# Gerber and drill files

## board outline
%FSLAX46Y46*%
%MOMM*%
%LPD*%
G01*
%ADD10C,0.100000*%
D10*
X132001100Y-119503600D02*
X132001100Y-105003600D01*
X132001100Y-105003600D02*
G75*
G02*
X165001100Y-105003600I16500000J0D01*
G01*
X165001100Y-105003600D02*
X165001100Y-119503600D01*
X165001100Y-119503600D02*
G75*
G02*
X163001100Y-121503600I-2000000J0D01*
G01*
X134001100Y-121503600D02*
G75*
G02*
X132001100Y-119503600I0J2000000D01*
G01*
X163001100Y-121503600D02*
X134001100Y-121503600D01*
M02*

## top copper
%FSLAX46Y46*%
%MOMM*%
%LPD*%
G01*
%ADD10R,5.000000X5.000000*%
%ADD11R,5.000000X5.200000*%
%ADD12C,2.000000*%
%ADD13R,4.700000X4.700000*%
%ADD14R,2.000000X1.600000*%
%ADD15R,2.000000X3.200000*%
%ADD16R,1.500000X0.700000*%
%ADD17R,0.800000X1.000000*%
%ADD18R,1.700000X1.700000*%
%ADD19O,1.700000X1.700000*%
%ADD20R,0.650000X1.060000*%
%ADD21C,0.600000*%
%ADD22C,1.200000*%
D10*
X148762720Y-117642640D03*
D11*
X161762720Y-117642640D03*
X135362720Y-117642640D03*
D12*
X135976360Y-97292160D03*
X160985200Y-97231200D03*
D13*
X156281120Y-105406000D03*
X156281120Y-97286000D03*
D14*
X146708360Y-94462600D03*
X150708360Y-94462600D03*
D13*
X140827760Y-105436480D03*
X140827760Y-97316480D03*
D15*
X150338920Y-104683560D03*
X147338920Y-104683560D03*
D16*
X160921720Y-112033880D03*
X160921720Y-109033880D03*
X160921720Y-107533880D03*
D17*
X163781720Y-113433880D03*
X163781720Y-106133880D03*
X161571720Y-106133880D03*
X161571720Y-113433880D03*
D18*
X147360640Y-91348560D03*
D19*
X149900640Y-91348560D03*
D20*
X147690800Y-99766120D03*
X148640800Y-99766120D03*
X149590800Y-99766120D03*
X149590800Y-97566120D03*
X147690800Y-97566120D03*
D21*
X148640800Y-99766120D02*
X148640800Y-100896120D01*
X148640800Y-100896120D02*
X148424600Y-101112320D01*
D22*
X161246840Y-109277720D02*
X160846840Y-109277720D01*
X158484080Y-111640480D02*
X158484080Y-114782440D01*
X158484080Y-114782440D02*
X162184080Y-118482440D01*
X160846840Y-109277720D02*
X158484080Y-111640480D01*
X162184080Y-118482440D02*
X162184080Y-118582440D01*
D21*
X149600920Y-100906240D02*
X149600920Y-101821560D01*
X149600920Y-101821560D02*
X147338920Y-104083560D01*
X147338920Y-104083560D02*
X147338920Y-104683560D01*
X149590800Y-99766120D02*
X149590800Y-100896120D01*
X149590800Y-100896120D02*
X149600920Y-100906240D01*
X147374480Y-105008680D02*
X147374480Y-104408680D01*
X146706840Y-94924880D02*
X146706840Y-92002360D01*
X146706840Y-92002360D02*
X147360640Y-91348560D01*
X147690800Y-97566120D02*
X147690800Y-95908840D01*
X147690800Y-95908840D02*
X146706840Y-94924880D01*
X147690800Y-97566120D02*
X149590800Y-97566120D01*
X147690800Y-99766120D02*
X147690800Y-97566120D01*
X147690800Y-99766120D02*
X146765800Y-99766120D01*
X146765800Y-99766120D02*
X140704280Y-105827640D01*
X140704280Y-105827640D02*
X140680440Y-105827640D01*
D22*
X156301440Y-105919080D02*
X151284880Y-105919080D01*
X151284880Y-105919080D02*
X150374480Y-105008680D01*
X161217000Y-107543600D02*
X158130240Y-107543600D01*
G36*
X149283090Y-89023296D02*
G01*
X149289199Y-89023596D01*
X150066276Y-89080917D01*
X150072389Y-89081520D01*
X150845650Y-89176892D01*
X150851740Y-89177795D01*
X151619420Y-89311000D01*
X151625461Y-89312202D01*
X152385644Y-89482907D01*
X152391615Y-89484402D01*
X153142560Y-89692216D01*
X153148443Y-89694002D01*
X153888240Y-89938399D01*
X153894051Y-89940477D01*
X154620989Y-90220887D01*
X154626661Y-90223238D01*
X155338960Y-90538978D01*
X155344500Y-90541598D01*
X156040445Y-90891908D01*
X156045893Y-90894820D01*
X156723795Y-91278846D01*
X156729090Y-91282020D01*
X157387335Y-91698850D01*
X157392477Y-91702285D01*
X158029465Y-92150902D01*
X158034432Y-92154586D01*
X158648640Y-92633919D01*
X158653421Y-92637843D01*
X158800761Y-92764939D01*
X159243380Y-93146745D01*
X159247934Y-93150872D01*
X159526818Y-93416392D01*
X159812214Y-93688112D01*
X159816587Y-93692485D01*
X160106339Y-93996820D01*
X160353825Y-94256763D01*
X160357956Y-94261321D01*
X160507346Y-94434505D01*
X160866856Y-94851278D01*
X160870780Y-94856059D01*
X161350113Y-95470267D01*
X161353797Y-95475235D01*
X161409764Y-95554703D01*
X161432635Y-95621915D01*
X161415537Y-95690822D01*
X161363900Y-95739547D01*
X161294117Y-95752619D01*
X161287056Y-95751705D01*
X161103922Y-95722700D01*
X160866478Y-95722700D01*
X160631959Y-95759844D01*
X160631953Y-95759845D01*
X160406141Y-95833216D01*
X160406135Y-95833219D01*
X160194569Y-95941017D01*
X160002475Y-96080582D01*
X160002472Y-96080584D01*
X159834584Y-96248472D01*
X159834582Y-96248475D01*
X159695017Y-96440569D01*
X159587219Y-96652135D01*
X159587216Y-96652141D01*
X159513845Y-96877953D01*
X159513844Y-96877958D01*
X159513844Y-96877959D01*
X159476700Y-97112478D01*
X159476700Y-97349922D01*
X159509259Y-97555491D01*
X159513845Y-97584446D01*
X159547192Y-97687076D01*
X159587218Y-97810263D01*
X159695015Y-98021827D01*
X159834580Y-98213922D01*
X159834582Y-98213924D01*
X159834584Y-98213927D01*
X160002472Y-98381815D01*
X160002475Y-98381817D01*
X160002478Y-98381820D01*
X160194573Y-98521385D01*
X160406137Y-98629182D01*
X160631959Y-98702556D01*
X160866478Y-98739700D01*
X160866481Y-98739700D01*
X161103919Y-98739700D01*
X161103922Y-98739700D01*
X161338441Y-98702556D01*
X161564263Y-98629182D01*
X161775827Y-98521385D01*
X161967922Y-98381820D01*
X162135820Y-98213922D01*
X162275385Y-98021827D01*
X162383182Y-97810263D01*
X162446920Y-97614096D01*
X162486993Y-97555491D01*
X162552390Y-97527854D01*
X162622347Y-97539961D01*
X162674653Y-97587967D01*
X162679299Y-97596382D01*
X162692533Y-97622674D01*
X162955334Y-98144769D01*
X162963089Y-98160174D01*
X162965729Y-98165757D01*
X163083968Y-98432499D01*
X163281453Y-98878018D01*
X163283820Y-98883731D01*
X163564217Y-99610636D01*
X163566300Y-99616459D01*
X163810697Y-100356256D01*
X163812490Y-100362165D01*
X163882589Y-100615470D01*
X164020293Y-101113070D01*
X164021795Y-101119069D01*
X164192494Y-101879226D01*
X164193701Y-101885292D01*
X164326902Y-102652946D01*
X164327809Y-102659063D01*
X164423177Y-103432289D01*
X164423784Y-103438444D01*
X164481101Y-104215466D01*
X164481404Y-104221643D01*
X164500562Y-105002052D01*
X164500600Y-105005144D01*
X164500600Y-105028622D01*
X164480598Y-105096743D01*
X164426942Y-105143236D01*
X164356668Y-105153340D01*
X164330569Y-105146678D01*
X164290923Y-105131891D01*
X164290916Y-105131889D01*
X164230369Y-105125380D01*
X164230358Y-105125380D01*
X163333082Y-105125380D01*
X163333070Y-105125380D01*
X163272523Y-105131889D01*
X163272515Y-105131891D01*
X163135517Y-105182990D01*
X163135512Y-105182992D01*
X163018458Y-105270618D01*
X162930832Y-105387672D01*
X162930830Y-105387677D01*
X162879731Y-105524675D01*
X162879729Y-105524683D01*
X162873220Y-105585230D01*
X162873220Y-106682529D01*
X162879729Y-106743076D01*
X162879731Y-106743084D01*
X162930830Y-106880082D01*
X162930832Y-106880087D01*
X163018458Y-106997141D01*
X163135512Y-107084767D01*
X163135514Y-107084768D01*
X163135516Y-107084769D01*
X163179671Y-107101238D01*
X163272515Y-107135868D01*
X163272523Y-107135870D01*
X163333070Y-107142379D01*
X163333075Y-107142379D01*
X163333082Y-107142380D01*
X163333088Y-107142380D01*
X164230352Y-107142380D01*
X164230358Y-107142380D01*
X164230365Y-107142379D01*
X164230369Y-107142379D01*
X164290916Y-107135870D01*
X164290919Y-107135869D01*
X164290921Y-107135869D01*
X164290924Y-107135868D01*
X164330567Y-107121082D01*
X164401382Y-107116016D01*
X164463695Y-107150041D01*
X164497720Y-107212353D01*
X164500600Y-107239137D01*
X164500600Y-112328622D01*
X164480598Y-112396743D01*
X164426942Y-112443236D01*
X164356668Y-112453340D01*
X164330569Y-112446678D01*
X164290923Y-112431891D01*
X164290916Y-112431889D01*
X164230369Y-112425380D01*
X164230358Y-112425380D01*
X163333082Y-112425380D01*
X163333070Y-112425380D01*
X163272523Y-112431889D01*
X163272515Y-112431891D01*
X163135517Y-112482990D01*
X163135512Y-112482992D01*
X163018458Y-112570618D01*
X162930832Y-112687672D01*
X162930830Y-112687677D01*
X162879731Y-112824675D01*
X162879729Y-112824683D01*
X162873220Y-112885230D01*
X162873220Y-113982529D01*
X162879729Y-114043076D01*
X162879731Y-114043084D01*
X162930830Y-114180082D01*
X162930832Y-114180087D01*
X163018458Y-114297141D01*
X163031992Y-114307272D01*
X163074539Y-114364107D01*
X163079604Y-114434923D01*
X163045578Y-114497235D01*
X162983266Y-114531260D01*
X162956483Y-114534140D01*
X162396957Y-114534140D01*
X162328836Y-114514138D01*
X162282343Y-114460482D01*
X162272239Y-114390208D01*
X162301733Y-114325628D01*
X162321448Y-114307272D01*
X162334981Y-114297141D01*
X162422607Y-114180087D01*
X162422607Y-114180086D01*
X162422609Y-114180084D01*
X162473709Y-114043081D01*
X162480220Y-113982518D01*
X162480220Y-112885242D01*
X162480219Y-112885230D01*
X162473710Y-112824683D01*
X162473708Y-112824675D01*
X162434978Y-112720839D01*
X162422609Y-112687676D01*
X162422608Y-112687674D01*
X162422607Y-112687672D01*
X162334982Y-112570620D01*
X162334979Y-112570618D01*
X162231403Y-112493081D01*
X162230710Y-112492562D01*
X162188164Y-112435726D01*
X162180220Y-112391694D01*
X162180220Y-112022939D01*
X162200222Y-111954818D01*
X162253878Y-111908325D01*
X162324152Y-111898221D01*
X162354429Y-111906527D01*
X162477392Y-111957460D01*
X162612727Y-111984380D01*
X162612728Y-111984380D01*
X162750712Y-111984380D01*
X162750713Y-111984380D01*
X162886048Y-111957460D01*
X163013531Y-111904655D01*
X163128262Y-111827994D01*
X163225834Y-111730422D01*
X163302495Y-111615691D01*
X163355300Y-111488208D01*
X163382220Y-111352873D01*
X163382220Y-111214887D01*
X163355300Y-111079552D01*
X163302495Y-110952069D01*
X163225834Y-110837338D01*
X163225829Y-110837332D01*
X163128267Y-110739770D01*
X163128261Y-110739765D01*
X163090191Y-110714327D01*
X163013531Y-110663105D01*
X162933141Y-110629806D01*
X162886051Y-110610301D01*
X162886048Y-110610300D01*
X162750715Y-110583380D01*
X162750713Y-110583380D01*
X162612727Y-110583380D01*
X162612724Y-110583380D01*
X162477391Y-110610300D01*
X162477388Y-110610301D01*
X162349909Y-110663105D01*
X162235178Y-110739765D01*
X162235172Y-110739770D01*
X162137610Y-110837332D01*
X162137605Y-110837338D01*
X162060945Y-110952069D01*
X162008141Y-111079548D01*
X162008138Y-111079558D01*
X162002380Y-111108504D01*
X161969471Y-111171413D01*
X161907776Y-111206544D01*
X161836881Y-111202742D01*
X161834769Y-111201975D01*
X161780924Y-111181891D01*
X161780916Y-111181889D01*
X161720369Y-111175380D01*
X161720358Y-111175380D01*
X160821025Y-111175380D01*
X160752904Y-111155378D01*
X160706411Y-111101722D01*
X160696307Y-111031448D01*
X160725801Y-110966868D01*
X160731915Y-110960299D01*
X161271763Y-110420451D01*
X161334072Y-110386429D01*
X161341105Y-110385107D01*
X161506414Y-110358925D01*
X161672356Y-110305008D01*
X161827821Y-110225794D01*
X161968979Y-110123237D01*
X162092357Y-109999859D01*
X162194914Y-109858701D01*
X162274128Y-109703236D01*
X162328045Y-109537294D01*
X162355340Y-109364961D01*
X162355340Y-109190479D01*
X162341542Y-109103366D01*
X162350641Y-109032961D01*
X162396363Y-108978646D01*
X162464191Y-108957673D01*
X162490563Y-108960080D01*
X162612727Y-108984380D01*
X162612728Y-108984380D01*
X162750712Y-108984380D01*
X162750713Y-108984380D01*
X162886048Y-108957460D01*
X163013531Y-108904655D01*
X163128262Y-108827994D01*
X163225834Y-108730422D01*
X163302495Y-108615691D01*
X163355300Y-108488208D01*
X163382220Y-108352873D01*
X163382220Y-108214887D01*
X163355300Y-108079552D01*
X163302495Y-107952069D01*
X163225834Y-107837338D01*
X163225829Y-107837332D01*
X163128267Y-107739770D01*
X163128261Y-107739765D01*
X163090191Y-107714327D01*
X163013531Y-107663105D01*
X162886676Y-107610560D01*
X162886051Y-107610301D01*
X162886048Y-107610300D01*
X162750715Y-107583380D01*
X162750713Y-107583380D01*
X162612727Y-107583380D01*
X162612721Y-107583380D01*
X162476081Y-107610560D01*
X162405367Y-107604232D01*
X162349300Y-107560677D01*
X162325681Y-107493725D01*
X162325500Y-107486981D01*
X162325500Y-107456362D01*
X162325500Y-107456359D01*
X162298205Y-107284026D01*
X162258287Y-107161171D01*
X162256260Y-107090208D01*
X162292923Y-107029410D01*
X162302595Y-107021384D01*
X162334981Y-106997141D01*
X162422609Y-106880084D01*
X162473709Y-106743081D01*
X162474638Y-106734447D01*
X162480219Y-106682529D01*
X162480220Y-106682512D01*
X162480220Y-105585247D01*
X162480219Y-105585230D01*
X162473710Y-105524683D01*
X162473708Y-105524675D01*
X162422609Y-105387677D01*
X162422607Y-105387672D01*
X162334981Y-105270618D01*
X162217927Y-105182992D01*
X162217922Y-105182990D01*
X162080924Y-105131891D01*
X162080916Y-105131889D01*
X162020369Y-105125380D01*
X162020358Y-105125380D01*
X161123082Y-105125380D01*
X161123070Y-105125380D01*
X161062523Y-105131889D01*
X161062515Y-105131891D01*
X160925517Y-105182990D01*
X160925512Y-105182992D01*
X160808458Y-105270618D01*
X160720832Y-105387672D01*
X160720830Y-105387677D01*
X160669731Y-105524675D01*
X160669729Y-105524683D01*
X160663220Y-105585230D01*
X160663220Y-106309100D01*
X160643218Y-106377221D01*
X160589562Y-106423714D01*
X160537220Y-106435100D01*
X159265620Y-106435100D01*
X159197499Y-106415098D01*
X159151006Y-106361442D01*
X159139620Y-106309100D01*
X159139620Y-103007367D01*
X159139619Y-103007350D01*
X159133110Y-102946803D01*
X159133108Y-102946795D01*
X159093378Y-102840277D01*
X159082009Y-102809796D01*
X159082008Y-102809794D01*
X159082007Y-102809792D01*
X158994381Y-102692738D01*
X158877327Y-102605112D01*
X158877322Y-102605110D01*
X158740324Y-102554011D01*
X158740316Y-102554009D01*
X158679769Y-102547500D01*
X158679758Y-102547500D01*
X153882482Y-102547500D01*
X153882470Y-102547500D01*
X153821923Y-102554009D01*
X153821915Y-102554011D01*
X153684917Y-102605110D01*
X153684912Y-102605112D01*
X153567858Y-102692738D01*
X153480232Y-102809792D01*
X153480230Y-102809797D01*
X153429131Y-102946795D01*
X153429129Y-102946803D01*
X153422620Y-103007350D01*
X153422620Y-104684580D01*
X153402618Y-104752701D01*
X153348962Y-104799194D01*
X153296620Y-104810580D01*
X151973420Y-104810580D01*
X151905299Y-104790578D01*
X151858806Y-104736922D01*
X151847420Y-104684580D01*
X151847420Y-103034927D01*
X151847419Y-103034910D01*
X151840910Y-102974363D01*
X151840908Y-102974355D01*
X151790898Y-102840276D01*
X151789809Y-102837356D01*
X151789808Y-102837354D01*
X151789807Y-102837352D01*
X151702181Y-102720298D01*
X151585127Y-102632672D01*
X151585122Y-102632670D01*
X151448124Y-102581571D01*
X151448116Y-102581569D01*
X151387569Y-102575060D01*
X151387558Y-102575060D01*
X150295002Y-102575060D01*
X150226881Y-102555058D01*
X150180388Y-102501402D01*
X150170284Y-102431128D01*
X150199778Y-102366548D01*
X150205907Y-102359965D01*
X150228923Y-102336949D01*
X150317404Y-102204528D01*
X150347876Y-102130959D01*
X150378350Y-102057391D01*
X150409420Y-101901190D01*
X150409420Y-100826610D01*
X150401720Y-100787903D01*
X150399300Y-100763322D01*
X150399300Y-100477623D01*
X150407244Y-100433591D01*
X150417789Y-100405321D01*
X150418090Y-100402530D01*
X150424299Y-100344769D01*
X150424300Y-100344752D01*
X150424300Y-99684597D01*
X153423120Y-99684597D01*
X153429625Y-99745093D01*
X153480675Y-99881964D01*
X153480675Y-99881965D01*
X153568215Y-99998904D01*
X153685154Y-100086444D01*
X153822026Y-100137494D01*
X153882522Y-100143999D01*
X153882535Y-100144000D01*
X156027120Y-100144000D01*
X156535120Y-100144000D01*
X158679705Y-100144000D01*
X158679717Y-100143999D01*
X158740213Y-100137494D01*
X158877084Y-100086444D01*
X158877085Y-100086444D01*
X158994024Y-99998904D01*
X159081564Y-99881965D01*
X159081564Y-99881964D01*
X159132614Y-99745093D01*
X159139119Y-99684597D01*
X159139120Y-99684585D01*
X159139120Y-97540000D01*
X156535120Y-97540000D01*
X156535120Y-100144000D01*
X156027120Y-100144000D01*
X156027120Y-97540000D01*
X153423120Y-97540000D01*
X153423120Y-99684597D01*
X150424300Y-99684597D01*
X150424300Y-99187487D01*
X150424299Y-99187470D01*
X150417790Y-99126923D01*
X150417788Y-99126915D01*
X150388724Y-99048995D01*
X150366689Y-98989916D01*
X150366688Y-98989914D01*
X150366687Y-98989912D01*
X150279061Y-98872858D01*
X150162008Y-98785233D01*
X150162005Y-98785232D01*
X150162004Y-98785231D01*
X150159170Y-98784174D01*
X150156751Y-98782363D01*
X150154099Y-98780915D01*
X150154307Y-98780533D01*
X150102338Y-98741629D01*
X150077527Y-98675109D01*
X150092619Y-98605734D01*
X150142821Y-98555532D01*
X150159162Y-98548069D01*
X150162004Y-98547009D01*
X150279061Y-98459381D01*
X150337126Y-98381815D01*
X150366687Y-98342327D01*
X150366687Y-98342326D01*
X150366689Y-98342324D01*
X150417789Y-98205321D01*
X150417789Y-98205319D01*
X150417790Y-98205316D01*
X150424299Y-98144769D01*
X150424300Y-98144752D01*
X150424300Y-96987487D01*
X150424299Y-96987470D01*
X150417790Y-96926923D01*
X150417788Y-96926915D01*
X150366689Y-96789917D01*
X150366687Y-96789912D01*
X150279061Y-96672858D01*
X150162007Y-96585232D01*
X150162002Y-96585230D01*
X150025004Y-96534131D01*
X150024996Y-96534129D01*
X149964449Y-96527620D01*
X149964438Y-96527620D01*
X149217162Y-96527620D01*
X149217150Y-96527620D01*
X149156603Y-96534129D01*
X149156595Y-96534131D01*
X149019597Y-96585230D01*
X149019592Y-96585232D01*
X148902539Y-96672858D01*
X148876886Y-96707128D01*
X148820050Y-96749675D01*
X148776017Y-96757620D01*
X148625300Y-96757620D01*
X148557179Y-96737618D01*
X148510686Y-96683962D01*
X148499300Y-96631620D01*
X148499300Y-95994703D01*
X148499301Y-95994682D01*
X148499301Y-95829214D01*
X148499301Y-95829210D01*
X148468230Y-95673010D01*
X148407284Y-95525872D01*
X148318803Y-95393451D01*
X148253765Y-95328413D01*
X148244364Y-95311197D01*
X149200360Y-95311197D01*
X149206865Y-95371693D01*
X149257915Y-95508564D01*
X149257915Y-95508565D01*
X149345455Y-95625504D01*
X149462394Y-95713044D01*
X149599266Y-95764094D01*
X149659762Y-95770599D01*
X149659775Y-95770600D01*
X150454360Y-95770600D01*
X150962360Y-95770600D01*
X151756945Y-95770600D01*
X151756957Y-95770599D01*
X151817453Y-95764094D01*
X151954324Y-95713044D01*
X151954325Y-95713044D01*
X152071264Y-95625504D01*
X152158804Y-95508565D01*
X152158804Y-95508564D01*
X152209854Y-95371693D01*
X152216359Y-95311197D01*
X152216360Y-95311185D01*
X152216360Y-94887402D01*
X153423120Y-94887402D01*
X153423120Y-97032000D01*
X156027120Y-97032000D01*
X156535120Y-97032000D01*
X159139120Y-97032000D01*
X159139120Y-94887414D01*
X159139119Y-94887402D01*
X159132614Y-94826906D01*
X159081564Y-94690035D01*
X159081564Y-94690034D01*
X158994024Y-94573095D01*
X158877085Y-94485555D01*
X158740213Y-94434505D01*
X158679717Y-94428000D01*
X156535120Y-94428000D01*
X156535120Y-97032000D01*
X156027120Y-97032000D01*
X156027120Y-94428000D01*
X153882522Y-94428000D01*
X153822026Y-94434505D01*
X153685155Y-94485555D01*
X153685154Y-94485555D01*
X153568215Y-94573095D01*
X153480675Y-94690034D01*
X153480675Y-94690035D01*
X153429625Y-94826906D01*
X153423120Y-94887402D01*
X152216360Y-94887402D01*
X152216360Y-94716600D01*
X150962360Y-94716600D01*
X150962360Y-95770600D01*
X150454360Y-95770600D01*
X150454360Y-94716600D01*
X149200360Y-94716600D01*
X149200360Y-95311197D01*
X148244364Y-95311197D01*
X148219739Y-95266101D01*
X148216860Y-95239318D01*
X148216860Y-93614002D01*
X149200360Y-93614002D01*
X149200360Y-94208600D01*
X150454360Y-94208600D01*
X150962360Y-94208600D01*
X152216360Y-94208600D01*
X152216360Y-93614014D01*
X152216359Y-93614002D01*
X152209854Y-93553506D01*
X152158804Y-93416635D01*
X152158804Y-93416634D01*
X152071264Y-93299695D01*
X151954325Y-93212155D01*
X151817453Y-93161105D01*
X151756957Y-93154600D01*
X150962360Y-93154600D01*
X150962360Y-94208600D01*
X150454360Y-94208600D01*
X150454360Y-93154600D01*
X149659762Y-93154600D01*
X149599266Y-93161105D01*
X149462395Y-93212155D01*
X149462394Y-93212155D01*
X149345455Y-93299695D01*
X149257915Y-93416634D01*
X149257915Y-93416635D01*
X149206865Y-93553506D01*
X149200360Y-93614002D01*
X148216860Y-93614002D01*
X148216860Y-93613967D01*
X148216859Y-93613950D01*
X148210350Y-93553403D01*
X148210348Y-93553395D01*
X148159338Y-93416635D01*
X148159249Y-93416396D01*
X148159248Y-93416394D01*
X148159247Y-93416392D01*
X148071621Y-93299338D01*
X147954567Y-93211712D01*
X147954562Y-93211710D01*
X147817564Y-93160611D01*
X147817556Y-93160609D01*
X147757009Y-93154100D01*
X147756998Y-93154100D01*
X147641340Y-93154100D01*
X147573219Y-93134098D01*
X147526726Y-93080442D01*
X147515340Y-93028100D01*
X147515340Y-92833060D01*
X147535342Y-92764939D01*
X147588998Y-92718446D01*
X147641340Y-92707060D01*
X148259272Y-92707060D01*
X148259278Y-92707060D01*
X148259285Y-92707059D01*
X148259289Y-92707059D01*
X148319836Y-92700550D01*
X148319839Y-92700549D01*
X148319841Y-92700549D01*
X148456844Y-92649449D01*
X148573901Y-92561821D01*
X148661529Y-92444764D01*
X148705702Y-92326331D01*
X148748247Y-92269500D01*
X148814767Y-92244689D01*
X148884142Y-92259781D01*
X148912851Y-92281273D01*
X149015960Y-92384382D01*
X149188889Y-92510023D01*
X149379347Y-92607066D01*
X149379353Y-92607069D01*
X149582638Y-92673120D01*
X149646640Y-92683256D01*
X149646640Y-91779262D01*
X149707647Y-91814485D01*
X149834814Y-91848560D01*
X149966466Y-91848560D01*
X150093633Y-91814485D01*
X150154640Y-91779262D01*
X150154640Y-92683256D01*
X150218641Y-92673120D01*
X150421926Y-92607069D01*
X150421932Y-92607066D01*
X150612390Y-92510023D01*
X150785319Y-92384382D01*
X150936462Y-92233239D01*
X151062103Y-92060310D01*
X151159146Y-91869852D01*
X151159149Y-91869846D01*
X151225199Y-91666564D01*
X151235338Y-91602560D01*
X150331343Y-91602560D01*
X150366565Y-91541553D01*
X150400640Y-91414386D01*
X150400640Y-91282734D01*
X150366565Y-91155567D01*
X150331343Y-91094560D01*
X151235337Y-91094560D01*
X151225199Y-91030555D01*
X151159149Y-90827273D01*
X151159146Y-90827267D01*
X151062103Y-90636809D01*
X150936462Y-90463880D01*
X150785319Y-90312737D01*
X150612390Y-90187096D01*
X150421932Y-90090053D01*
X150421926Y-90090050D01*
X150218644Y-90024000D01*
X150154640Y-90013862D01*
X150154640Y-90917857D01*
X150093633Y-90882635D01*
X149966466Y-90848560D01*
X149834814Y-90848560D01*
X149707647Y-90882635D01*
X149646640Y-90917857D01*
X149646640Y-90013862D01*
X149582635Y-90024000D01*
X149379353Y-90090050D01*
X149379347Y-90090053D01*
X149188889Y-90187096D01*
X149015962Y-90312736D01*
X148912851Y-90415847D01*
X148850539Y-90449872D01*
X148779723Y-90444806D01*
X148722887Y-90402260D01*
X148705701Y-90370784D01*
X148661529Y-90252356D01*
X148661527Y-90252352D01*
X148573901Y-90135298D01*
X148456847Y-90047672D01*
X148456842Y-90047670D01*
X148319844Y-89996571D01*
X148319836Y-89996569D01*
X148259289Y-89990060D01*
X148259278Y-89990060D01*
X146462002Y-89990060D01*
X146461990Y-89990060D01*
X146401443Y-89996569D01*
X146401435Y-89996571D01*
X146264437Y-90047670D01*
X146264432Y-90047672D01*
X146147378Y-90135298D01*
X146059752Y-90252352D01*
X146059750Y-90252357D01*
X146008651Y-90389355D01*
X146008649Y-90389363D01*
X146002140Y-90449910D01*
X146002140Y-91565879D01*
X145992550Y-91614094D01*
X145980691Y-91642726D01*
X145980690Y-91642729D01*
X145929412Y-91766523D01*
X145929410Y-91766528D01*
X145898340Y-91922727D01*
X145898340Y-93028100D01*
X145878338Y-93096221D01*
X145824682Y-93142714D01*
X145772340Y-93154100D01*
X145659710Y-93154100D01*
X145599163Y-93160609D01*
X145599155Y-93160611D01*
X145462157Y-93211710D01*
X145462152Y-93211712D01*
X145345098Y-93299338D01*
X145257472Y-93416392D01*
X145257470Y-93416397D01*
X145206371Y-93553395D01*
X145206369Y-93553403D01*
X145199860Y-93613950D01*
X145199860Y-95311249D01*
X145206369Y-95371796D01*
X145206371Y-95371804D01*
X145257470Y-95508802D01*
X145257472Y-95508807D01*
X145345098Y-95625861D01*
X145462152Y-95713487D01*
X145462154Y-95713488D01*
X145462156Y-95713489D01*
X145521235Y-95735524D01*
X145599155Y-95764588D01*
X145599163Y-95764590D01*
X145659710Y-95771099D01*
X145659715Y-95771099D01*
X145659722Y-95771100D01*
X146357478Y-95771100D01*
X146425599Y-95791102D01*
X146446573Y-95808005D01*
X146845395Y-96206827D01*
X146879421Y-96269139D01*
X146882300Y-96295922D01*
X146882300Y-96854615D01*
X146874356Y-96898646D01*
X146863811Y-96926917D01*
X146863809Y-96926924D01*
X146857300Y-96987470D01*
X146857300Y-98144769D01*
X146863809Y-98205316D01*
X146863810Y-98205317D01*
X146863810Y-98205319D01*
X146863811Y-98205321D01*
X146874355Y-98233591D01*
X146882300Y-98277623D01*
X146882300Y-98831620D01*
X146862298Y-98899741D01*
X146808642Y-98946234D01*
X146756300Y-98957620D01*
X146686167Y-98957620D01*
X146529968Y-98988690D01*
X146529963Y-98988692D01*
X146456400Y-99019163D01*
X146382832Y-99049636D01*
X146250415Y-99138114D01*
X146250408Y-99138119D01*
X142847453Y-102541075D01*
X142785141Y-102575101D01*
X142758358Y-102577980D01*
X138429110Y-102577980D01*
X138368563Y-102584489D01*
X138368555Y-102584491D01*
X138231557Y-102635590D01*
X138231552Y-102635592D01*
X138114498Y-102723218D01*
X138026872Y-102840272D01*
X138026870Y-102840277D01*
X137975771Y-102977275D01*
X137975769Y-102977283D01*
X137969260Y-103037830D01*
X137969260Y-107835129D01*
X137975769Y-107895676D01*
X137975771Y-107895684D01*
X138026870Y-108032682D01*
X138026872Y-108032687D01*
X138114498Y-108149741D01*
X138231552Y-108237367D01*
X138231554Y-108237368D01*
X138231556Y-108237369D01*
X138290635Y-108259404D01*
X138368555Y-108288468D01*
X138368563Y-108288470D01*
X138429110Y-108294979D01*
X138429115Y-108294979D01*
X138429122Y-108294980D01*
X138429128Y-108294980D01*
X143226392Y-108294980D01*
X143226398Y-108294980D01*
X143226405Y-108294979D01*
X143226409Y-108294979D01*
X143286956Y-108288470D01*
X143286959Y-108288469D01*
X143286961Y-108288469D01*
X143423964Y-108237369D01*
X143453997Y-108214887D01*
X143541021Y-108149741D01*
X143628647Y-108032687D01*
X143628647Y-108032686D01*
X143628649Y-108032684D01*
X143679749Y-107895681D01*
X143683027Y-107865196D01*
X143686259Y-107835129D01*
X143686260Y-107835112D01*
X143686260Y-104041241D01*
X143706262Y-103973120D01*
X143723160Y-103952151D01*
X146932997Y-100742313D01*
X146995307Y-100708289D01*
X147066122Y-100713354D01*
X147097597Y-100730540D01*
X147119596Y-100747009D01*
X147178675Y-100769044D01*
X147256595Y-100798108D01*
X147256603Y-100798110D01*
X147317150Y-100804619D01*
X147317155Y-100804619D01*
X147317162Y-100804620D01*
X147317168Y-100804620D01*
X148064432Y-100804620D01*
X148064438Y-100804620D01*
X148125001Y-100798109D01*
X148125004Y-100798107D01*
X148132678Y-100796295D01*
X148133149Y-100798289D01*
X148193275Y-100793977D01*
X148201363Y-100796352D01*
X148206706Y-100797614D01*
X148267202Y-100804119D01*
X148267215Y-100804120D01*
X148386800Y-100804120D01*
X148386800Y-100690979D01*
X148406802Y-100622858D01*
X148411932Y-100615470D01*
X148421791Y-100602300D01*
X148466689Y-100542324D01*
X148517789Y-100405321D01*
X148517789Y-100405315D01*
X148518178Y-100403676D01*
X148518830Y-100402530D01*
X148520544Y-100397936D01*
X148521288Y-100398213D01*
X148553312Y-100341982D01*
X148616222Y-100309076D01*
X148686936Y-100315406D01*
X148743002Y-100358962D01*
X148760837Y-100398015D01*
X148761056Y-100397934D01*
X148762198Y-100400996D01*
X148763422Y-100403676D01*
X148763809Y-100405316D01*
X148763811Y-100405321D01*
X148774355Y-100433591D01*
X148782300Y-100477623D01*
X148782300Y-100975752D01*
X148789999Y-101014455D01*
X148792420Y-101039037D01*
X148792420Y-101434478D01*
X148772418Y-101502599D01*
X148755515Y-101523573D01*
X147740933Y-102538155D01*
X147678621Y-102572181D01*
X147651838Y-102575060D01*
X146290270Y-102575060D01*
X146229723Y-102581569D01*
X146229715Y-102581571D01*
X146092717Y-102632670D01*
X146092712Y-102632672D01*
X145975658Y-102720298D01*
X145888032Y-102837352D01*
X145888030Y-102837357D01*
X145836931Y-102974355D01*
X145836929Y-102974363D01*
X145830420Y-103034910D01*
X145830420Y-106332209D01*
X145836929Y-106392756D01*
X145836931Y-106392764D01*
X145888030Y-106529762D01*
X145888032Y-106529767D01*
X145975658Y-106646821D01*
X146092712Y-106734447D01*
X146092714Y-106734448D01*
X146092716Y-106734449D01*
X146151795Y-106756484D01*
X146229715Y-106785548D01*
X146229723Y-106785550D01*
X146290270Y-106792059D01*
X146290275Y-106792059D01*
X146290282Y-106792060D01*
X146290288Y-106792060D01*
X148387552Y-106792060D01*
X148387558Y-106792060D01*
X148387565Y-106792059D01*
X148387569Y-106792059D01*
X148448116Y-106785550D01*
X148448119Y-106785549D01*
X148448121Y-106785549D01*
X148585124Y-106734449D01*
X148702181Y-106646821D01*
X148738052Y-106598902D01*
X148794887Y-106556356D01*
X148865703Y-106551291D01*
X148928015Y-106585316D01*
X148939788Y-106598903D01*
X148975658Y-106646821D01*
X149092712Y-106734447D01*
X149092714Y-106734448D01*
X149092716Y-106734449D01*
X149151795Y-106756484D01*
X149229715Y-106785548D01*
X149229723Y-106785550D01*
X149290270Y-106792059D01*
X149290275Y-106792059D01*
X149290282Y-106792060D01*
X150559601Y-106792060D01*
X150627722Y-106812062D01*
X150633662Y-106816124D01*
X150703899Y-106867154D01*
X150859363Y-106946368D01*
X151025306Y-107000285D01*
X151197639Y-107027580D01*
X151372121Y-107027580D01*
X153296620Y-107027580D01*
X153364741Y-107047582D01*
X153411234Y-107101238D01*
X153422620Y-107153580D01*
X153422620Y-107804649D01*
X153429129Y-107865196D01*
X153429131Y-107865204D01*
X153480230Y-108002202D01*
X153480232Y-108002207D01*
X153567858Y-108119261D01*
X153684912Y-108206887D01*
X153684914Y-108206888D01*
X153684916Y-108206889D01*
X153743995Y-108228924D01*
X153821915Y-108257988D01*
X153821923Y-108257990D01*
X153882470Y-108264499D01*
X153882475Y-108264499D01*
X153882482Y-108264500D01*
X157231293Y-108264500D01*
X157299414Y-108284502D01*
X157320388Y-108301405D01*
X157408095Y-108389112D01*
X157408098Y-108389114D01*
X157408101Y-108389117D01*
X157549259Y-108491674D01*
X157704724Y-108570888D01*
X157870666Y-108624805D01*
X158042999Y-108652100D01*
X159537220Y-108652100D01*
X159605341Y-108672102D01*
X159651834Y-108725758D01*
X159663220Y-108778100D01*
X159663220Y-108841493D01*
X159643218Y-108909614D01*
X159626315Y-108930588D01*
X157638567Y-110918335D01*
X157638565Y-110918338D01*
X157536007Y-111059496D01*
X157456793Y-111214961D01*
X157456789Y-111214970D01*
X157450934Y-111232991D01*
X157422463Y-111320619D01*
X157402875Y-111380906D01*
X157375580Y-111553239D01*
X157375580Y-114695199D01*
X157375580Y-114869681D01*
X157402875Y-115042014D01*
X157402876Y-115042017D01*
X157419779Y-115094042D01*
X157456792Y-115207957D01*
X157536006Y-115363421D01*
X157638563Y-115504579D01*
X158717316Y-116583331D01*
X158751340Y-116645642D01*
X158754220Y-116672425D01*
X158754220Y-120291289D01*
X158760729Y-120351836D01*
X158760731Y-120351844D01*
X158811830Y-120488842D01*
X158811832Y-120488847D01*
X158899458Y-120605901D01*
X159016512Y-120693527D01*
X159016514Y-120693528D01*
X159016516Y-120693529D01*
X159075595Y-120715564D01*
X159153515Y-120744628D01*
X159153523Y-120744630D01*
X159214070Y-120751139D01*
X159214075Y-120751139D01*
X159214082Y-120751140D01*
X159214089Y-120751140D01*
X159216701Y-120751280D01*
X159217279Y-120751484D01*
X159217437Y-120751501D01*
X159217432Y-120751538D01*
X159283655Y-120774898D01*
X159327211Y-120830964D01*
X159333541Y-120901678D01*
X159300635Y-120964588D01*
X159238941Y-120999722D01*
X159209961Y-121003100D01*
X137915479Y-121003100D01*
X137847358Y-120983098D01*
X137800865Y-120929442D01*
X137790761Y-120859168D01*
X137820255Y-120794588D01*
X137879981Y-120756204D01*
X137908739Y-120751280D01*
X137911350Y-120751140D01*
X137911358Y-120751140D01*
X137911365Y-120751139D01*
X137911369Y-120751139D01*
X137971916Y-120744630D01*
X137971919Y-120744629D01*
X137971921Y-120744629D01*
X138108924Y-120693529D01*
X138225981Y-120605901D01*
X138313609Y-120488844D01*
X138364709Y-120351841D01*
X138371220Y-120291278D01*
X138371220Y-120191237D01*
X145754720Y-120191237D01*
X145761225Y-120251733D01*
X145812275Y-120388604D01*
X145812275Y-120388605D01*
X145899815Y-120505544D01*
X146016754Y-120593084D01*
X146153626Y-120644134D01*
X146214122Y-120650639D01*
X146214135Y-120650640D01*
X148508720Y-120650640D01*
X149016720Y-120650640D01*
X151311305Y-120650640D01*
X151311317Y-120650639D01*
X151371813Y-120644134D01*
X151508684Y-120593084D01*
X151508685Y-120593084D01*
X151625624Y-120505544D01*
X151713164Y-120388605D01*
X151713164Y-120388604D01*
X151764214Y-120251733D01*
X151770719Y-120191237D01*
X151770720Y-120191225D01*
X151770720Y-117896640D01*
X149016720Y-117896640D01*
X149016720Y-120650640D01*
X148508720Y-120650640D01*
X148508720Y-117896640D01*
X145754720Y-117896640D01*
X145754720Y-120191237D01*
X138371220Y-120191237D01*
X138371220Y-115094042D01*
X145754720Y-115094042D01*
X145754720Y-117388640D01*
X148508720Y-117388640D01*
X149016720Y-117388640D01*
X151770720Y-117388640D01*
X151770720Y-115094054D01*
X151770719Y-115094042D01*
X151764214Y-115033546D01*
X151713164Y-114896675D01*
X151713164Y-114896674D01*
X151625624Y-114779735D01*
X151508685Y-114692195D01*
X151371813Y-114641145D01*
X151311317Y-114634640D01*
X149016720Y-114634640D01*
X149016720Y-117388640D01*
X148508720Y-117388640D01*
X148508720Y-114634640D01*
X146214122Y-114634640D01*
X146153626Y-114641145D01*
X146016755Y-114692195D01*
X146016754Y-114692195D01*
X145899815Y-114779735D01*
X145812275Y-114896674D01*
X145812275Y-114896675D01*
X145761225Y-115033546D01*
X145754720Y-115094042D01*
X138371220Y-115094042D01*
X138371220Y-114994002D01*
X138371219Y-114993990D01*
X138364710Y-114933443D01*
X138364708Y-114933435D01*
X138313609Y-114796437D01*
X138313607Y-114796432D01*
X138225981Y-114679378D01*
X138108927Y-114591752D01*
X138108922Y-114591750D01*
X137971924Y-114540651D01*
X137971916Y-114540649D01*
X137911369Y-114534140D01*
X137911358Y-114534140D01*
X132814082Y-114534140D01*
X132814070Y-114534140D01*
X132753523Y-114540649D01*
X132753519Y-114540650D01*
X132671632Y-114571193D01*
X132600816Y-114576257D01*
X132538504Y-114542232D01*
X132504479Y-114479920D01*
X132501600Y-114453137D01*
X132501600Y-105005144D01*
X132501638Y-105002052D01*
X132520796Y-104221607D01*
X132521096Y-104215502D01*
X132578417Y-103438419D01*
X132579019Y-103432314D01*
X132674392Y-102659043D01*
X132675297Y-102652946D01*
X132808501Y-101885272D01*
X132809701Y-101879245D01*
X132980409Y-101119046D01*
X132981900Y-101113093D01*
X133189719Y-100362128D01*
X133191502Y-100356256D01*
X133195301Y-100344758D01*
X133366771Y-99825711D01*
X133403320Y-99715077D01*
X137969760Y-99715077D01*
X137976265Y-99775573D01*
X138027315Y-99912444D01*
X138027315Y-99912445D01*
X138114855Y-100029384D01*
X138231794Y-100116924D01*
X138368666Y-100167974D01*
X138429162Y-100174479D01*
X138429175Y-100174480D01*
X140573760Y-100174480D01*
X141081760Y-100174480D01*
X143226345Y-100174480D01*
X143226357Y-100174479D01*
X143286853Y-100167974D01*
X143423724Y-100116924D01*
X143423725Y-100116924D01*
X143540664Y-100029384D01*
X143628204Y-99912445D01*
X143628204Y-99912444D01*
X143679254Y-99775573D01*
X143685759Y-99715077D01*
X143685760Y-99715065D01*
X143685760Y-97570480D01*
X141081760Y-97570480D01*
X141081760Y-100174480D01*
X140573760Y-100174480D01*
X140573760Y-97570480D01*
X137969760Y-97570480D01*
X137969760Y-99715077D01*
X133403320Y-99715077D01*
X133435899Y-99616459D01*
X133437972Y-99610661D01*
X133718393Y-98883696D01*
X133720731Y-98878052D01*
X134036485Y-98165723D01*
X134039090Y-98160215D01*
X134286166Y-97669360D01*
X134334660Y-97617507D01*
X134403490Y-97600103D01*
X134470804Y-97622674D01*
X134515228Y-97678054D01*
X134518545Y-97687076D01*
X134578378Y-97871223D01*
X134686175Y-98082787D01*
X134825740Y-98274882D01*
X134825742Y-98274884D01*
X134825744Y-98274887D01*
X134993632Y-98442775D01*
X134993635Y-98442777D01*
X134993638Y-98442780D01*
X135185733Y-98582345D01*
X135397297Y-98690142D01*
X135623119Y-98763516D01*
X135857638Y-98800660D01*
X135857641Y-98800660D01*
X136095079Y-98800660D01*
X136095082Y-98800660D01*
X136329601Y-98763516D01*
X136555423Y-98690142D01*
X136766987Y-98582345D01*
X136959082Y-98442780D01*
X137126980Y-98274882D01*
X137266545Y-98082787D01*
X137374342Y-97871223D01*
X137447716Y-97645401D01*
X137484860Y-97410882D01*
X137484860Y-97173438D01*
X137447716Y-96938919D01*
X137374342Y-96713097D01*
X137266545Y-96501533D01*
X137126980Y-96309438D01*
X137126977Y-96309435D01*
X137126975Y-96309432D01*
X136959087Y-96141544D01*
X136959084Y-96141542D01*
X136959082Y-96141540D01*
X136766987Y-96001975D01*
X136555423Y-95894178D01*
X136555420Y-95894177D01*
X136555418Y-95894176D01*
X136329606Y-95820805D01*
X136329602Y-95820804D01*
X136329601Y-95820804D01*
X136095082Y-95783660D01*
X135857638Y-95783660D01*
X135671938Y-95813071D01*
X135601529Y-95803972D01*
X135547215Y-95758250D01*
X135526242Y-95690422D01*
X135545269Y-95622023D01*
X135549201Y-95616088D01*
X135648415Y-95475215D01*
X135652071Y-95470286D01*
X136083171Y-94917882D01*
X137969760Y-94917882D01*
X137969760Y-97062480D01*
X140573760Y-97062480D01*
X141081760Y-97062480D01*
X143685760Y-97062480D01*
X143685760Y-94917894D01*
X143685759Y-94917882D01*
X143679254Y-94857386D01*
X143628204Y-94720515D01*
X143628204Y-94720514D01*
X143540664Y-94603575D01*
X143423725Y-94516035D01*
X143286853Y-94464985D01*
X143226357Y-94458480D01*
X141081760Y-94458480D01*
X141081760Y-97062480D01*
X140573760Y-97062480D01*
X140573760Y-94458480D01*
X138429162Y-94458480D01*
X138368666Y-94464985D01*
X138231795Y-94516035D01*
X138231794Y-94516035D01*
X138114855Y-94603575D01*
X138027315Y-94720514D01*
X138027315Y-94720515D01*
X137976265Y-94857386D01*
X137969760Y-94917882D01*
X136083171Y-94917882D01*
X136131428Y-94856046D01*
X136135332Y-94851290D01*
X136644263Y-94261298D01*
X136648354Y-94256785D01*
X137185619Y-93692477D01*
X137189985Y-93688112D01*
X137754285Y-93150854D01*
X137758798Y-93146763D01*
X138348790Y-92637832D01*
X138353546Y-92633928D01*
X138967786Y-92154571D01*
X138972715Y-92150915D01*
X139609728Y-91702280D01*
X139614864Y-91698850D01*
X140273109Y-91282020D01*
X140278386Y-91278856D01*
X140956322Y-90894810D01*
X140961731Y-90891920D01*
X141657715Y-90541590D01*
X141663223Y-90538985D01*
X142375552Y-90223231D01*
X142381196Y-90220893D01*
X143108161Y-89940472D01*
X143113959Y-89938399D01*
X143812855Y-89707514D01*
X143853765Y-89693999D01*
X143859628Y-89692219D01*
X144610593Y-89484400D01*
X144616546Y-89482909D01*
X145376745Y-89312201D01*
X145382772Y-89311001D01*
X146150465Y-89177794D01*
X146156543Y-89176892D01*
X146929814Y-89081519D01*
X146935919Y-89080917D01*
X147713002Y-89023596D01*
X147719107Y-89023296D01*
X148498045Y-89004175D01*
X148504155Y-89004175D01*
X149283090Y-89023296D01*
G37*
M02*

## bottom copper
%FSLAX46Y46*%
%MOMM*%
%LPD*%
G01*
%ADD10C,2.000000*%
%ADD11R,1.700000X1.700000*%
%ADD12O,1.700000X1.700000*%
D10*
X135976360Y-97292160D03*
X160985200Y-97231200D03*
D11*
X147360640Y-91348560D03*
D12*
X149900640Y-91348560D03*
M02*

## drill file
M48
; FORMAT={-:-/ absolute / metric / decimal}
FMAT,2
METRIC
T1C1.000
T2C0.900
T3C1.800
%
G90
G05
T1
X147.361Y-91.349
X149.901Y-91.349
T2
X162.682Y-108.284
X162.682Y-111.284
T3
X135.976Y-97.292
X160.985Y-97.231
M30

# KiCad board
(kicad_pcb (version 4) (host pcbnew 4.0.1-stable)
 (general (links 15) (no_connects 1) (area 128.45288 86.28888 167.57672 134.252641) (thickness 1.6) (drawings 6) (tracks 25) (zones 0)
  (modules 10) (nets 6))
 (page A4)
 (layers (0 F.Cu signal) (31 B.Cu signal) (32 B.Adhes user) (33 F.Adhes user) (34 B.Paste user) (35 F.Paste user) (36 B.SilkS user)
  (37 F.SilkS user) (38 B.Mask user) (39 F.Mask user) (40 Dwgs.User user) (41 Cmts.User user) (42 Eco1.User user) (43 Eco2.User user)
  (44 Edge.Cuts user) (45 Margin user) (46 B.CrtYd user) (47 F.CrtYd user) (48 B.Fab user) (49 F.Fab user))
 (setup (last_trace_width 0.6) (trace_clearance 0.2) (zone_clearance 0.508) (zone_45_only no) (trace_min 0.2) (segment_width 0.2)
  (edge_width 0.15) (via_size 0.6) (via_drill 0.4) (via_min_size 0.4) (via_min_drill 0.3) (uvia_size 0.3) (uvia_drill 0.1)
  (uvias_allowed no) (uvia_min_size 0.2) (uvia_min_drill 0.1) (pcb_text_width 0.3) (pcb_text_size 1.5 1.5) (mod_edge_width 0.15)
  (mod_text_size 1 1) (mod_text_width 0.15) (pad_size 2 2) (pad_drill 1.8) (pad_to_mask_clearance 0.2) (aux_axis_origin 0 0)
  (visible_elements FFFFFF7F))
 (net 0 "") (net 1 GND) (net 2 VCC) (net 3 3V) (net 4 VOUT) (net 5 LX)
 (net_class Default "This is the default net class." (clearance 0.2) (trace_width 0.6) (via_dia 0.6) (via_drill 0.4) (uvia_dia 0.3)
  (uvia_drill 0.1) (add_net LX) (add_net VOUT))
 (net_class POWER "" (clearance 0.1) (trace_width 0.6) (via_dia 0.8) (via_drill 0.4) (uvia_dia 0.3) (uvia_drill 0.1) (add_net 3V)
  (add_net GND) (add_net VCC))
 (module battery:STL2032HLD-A (layer F.Cu) (at 148.76272 117.64264)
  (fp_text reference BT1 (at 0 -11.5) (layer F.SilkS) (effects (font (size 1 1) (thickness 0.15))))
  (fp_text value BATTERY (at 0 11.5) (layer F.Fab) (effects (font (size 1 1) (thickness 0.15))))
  (pad 2 smd rect (at 0 0) (size 5 5) (layers F.Cu F.Paste F.Mask) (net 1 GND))
  (pad 1 smd rect (at 13 0) (size 5 5.2) (layers F.Cu F.Paste F.Mask) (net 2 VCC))
  (pad 1 smd rect (at -13.4 0) (size 5 5.2) (layers F.Cu F.Paste F.Mask) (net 2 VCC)))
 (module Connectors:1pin (layer F.Cu) (at 135.97636 97.29216)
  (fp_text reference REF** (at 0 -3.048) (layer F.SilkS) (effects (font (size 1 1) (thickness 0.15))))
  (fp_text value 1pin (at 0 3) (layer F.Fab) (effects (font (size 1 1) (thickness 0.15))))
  (pad "" np_thru_hole circle (at 0 0) (size 2 2) (drill 1.8) (layers *.Cu *.Mask F.SilkS)))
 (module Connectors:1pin (layer F.Cu) (at 160.9852 97.2312)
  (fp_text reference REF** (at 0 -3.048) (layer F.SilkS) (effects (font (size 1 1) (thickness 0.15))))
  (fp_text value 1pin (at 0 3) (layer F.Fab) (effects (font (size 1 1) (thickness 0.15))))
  (pad "" np_thru_hole circle (at 0 0) (size 2 2) (drill 1.8) (layers *.Cu *.Mask F.SilkS)))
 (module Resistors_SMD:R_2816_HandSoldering (layer F.Cu) (at 156.28112 101.346 90)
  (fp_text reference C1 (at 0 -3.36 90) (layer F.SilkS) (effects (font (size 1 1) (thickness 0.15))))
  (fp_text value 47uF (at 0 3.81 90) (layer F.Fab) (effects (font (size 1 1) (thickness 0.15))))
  (pad 1 smd rect (at -4.06 0 90) (size 4.7 4.7) (layers F.Cu F.Paste F.Mask) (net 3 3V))
  (pad 2 smd rect (at 4.06 0 90) (size 4.7 4.7) (layers F.Cu F.Paste F.Mask) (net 1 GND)))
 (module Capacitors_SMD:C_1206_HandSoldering (layer F.Cu) (at 148.70836 94.4626)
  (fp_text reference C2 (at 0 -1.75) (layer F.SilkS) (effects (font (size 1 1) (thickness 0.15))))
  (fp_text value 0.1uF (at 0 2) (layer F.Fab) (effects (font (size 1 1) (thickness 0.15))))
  (pad 1 smd rect (at -2 0) (size 2 1.6) (layers F.Cu F.Paste F.Mask) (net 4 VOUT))
  (pad 2 smd rect (at 2 0) (size 2 1.6) (layers F.Cu F.Paste F.Mask) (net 1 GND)))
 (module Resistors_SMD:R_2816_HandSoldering (layer F.Cu) (at 140.82776 101.37648 90)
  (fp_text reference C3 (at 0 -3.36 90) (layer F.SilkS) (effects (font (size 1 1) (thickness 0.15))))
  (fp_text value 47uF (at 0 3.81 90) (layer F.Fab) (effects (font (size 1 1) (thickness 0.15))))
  (pad 1 smd rect (at -4.06 0 90) (size 4.7 4.7) (layers F.Cu F.Paste F.Mask) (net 4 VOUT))
  (pad 2 smd rect (at 4.06 0 90) (size 4.7 4.7) (layers F.Cu F.Paste F.Mask) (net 1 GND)))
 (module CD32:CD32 (layer F.Cu) (at 148.83892 104.68356 90)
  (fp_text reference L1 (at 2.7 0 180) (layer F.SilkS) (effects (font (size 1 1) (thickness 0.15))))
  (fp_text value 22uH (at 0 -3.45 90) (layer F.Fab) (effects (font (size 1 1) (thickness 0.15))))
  (pad 2 smd rect (at 0 1.5 90) (size 3.2 2) (layers F.Cu F.Paste F.Mask) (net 3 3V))
  (pad 1 smd rect (at 0 -1.5 90) (size 3.2 2) (layers F.Cu F.Paste F.Mask) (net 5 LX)))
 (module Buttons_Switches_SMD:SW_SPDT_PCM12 (layer F.Cu) (at 162.35172 109.78388 90)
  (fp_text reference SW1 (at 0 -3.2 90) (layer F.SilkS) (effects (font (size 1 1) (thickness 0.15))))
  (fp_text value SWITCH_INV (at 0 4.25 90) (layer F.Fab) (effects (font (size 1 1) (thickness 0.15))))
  (pad "" np_thru_hole circle (at -1.5 0.33 90) (size 0.9 0.9) (drill 0.9) (layers *.Cu *.Mask))
  (pad "" np_thru_hole circle (at 1.5 0.33 90) (size 0.9 0.9) (drill 0.9) (layers *.Cu *.Mask))
  (pad 1 smd rect (at -2.25 -1.43 90) (size 0.7 1.5) (layers F.Cu F.Paste F.Mask))
  (pad 2 smd rect (at 0.75 -1.43 90) (size 0.7 1.5) (layers F.Cu F.Paste F.Mask) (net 2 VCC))
  (pad 3 smd rect (at 2.25 -1.43 90) (size 0.7 1.5) (layers F.Cu F.Paste F.Mask) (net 3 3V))
  (pad "" smd rect (at -3.65 1.43 90) (size 1 0.8) (layers F.Cu F.Paste F.Mask))
  (pad "" smd rect (at 3.65 1.43 90) (size 1 0.8) (layers F.Cu F.Paste F.Mask))
  (pad "" smd rect (at 3.65 -0.78 90) (size 1 0.8) (layers F.Cu F.Paste F.Mask))
  (pad "" smd rect (at -3.65 -0.78 90) (size 1 0.8) (layers F.Cu F.Paste F.Mask)))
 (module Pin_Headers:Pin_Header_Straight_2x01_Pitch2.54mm (layer F.Cu) (at 147.36064 91.34856)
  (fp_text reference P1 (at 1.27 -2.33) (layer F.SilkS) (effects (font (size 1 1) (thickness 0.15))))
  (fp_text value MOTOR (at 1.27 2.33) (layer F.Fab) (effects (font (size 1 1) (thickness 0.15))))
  (pad 1 thru_hole rect (at 0 0) (size 1.7 1.7) (drill 1) (layers *.Cu *.Mask) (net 4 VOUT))
  (pad 2 thru_hole oval (at 2.54 0) (size 1.7 1.7) (drill 1) (layers *.Cu *.Mask) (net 1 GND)))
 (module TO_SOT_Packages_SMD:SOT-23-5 (layer F.Cu) (at 148.6408 98.66612 90)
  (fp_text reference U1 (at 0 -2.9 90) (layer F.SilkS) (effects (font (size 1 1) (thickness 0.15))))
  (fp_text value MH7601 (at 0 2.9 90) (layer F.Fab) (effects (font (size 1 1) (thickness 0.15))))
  (pad 1 smd rect (at -1.1 -0.95 90) (size 1.06 0.65) (layers F.Cu F.Paste F.Mask) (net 4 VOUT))
  (pad 2 smd rect (at -1.1 0 90) (size 1.06 0.65) (layers F.Cu F.Paste F.Mask) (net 1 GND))
  (pad 3 smd rect (at -1.1 0.95 90) (size 1.06 0.65) (layers F.Cu F.Paste F.Mask) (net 5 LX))
  (pad 4 smd rect (at 1.1 0.95 90) (size 1.06 0.65) (layers F.Cu F.Paste F.Mask) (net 4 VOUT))
  (pad 5 smd rect (at 1.1 -0.95 90) (size 1.06 0.65) (layers F.Cu F.Paste F.Mask) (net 4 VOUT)))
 (gr_line (start 132.0011 119.5036) (end 132.0011 105.0036) (layer Edge.Cuts) (width 0.1))
 (gr_arc (start 148.5011 105.0036) (end 165.0011 105.0036) (angle -180) (layer Edge.Cuts) (width 0.1))
 (gr_line (start 165.0011 105.0036) (end 165.0011 119.5036) (layer Edge.Cuts) (width 0.1))
 (gr_arc (start 163.0011 119.5036) (end 163.0011 121.5036) (angle -90) (layer Edge.Cuts) (width 0.1))
 (gr_arc (start 134.0011 119.5036) (end 132.0011 119.5036) (angle -90) (layer Edge.Cuts) (width 0.1))
 (gr_line (start 163.0011 121.5036) (end 134.0011 121.5036) (layer Edge.Cuts) (width 0.1))
 (segment (start 148.6408 99.76612) (end 148.6408 100.89612) (width 0.6) (layer F.Cu) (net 1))
 (segment (start 148.6408 100.89612) (end 148.4246 101.11232) (width 0.6) (layer F.Cu) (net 1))
 (segment (start 161.24684 109.27772) (end 160.84684 109.27772) (width 1.2) (layer F.Cu) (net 2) (status 30))
 (segment (start 158.48408 111.64048) (end 158.48408 114.78244) (width 1.2) (layer F.Cu) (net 2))
 (segment (start 158.48408 114.78244) (end 162.18408 118.48244) (width 1.2) (layer F.Cu) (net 2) (status 20))
 (segment (start 160.84684 109.27772) (end 158.48408 111.64048) (width 1.2) (layer F.Cu) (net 2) (status 10))
 (segment (start 162.18408 118.48244) (end 162.18408 118.58244) (width 1.2) (layer F.Cu) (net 2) (status 30))
 (segment (start 149.60092 100.90624) (end 149.60092 101.82156) (width 0.6) (layer F.Cu) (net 5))
 (segment (start 149.60092 101.82156) (end 147.33892 104.08356) (width 0.6) (layer F.Cu) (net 5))
 (segment (start 147.33892 104.08356) (end 147.33892 104.68356) (width 0.6) (layer F.Cu) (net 5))
 (segment (start 149.5908 99.76612) (end 149.5908 100.89612) (width 0.6) (layer F.Cu) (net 5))
 (segment (start 149.5908 100.89612) (end 149.60092 100.90624) (width 0.6) (layer F.Cu) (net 5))
 (segment (start 147.37448 105.00868) (end 147.37448 104.40868) (width 0.6) (layer F.Cu) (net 5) (status 30))
 (segment (start 146.70684 94.92488) (end 146.70684 92.00236) (width 0.6) (layer F.Cu) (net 4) (status 30))
 (segment (start 146.70684 92.00236) (end 147.36064 91.34856) (width 0.6) (layer F.Cu) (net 4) (status 30))
 (segment (start 147.6908 97.56612) (end 147.6908 95.90884) (width 0.6) (layer F.Cu) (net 4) (status 10))
 (segment (start 147.6908 95.90884) (end 146.70684 94.92488) (width 0.6) (layer F.Cu) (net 4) (status 20))
 (segment (start 147.6908 97.56612) (end 149.5908 97.56612) (width 0.6) (layer F.Cu) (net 4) (status 30))
 (segment (start 147.6908 99.76612) (end 147.6908 97.56612) (width 0.6) (layer F.Cu) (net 4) (status 30))
 (segment (start 147.6908 99.76612) (end 146.7658 99.76612) (width 0.6) (layer F.Cu) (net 4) (status 10))
 (segment (start 146.7658 99.76612) (end 140.70428 105.82764) (width 0.6) (layer F.Cu) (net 4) (status 20))
 (segment (start 140.70428 105.82764) (end 140.68044 105.82764) (width 0.6) (layer F.Cu) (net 4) (status 30))
 (segment (start 156.30144 105.91908) (end 151.28488 105.91908) (width 1.2) (layer F.Cu) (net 3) (status 30))
 (segment (start 151.28488 105.91908) (end 150.37448 105.00868) (width 1.2) (layer F.Cu) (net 3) (status 30))
 (segment (start 161.217 107.5436) (end 158.13024 107.5436) (width 1.2) (layer F.Cu) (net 3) (status 30))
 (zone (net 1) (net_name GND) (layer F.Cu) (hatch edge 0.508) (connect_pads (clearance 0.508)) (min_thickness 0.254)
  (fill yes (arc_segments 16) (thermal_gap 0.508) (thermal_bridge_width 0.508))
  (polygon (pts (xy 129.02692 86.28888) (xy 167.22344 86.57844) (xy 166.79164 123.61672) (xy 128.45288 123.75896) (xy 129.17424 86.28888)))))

